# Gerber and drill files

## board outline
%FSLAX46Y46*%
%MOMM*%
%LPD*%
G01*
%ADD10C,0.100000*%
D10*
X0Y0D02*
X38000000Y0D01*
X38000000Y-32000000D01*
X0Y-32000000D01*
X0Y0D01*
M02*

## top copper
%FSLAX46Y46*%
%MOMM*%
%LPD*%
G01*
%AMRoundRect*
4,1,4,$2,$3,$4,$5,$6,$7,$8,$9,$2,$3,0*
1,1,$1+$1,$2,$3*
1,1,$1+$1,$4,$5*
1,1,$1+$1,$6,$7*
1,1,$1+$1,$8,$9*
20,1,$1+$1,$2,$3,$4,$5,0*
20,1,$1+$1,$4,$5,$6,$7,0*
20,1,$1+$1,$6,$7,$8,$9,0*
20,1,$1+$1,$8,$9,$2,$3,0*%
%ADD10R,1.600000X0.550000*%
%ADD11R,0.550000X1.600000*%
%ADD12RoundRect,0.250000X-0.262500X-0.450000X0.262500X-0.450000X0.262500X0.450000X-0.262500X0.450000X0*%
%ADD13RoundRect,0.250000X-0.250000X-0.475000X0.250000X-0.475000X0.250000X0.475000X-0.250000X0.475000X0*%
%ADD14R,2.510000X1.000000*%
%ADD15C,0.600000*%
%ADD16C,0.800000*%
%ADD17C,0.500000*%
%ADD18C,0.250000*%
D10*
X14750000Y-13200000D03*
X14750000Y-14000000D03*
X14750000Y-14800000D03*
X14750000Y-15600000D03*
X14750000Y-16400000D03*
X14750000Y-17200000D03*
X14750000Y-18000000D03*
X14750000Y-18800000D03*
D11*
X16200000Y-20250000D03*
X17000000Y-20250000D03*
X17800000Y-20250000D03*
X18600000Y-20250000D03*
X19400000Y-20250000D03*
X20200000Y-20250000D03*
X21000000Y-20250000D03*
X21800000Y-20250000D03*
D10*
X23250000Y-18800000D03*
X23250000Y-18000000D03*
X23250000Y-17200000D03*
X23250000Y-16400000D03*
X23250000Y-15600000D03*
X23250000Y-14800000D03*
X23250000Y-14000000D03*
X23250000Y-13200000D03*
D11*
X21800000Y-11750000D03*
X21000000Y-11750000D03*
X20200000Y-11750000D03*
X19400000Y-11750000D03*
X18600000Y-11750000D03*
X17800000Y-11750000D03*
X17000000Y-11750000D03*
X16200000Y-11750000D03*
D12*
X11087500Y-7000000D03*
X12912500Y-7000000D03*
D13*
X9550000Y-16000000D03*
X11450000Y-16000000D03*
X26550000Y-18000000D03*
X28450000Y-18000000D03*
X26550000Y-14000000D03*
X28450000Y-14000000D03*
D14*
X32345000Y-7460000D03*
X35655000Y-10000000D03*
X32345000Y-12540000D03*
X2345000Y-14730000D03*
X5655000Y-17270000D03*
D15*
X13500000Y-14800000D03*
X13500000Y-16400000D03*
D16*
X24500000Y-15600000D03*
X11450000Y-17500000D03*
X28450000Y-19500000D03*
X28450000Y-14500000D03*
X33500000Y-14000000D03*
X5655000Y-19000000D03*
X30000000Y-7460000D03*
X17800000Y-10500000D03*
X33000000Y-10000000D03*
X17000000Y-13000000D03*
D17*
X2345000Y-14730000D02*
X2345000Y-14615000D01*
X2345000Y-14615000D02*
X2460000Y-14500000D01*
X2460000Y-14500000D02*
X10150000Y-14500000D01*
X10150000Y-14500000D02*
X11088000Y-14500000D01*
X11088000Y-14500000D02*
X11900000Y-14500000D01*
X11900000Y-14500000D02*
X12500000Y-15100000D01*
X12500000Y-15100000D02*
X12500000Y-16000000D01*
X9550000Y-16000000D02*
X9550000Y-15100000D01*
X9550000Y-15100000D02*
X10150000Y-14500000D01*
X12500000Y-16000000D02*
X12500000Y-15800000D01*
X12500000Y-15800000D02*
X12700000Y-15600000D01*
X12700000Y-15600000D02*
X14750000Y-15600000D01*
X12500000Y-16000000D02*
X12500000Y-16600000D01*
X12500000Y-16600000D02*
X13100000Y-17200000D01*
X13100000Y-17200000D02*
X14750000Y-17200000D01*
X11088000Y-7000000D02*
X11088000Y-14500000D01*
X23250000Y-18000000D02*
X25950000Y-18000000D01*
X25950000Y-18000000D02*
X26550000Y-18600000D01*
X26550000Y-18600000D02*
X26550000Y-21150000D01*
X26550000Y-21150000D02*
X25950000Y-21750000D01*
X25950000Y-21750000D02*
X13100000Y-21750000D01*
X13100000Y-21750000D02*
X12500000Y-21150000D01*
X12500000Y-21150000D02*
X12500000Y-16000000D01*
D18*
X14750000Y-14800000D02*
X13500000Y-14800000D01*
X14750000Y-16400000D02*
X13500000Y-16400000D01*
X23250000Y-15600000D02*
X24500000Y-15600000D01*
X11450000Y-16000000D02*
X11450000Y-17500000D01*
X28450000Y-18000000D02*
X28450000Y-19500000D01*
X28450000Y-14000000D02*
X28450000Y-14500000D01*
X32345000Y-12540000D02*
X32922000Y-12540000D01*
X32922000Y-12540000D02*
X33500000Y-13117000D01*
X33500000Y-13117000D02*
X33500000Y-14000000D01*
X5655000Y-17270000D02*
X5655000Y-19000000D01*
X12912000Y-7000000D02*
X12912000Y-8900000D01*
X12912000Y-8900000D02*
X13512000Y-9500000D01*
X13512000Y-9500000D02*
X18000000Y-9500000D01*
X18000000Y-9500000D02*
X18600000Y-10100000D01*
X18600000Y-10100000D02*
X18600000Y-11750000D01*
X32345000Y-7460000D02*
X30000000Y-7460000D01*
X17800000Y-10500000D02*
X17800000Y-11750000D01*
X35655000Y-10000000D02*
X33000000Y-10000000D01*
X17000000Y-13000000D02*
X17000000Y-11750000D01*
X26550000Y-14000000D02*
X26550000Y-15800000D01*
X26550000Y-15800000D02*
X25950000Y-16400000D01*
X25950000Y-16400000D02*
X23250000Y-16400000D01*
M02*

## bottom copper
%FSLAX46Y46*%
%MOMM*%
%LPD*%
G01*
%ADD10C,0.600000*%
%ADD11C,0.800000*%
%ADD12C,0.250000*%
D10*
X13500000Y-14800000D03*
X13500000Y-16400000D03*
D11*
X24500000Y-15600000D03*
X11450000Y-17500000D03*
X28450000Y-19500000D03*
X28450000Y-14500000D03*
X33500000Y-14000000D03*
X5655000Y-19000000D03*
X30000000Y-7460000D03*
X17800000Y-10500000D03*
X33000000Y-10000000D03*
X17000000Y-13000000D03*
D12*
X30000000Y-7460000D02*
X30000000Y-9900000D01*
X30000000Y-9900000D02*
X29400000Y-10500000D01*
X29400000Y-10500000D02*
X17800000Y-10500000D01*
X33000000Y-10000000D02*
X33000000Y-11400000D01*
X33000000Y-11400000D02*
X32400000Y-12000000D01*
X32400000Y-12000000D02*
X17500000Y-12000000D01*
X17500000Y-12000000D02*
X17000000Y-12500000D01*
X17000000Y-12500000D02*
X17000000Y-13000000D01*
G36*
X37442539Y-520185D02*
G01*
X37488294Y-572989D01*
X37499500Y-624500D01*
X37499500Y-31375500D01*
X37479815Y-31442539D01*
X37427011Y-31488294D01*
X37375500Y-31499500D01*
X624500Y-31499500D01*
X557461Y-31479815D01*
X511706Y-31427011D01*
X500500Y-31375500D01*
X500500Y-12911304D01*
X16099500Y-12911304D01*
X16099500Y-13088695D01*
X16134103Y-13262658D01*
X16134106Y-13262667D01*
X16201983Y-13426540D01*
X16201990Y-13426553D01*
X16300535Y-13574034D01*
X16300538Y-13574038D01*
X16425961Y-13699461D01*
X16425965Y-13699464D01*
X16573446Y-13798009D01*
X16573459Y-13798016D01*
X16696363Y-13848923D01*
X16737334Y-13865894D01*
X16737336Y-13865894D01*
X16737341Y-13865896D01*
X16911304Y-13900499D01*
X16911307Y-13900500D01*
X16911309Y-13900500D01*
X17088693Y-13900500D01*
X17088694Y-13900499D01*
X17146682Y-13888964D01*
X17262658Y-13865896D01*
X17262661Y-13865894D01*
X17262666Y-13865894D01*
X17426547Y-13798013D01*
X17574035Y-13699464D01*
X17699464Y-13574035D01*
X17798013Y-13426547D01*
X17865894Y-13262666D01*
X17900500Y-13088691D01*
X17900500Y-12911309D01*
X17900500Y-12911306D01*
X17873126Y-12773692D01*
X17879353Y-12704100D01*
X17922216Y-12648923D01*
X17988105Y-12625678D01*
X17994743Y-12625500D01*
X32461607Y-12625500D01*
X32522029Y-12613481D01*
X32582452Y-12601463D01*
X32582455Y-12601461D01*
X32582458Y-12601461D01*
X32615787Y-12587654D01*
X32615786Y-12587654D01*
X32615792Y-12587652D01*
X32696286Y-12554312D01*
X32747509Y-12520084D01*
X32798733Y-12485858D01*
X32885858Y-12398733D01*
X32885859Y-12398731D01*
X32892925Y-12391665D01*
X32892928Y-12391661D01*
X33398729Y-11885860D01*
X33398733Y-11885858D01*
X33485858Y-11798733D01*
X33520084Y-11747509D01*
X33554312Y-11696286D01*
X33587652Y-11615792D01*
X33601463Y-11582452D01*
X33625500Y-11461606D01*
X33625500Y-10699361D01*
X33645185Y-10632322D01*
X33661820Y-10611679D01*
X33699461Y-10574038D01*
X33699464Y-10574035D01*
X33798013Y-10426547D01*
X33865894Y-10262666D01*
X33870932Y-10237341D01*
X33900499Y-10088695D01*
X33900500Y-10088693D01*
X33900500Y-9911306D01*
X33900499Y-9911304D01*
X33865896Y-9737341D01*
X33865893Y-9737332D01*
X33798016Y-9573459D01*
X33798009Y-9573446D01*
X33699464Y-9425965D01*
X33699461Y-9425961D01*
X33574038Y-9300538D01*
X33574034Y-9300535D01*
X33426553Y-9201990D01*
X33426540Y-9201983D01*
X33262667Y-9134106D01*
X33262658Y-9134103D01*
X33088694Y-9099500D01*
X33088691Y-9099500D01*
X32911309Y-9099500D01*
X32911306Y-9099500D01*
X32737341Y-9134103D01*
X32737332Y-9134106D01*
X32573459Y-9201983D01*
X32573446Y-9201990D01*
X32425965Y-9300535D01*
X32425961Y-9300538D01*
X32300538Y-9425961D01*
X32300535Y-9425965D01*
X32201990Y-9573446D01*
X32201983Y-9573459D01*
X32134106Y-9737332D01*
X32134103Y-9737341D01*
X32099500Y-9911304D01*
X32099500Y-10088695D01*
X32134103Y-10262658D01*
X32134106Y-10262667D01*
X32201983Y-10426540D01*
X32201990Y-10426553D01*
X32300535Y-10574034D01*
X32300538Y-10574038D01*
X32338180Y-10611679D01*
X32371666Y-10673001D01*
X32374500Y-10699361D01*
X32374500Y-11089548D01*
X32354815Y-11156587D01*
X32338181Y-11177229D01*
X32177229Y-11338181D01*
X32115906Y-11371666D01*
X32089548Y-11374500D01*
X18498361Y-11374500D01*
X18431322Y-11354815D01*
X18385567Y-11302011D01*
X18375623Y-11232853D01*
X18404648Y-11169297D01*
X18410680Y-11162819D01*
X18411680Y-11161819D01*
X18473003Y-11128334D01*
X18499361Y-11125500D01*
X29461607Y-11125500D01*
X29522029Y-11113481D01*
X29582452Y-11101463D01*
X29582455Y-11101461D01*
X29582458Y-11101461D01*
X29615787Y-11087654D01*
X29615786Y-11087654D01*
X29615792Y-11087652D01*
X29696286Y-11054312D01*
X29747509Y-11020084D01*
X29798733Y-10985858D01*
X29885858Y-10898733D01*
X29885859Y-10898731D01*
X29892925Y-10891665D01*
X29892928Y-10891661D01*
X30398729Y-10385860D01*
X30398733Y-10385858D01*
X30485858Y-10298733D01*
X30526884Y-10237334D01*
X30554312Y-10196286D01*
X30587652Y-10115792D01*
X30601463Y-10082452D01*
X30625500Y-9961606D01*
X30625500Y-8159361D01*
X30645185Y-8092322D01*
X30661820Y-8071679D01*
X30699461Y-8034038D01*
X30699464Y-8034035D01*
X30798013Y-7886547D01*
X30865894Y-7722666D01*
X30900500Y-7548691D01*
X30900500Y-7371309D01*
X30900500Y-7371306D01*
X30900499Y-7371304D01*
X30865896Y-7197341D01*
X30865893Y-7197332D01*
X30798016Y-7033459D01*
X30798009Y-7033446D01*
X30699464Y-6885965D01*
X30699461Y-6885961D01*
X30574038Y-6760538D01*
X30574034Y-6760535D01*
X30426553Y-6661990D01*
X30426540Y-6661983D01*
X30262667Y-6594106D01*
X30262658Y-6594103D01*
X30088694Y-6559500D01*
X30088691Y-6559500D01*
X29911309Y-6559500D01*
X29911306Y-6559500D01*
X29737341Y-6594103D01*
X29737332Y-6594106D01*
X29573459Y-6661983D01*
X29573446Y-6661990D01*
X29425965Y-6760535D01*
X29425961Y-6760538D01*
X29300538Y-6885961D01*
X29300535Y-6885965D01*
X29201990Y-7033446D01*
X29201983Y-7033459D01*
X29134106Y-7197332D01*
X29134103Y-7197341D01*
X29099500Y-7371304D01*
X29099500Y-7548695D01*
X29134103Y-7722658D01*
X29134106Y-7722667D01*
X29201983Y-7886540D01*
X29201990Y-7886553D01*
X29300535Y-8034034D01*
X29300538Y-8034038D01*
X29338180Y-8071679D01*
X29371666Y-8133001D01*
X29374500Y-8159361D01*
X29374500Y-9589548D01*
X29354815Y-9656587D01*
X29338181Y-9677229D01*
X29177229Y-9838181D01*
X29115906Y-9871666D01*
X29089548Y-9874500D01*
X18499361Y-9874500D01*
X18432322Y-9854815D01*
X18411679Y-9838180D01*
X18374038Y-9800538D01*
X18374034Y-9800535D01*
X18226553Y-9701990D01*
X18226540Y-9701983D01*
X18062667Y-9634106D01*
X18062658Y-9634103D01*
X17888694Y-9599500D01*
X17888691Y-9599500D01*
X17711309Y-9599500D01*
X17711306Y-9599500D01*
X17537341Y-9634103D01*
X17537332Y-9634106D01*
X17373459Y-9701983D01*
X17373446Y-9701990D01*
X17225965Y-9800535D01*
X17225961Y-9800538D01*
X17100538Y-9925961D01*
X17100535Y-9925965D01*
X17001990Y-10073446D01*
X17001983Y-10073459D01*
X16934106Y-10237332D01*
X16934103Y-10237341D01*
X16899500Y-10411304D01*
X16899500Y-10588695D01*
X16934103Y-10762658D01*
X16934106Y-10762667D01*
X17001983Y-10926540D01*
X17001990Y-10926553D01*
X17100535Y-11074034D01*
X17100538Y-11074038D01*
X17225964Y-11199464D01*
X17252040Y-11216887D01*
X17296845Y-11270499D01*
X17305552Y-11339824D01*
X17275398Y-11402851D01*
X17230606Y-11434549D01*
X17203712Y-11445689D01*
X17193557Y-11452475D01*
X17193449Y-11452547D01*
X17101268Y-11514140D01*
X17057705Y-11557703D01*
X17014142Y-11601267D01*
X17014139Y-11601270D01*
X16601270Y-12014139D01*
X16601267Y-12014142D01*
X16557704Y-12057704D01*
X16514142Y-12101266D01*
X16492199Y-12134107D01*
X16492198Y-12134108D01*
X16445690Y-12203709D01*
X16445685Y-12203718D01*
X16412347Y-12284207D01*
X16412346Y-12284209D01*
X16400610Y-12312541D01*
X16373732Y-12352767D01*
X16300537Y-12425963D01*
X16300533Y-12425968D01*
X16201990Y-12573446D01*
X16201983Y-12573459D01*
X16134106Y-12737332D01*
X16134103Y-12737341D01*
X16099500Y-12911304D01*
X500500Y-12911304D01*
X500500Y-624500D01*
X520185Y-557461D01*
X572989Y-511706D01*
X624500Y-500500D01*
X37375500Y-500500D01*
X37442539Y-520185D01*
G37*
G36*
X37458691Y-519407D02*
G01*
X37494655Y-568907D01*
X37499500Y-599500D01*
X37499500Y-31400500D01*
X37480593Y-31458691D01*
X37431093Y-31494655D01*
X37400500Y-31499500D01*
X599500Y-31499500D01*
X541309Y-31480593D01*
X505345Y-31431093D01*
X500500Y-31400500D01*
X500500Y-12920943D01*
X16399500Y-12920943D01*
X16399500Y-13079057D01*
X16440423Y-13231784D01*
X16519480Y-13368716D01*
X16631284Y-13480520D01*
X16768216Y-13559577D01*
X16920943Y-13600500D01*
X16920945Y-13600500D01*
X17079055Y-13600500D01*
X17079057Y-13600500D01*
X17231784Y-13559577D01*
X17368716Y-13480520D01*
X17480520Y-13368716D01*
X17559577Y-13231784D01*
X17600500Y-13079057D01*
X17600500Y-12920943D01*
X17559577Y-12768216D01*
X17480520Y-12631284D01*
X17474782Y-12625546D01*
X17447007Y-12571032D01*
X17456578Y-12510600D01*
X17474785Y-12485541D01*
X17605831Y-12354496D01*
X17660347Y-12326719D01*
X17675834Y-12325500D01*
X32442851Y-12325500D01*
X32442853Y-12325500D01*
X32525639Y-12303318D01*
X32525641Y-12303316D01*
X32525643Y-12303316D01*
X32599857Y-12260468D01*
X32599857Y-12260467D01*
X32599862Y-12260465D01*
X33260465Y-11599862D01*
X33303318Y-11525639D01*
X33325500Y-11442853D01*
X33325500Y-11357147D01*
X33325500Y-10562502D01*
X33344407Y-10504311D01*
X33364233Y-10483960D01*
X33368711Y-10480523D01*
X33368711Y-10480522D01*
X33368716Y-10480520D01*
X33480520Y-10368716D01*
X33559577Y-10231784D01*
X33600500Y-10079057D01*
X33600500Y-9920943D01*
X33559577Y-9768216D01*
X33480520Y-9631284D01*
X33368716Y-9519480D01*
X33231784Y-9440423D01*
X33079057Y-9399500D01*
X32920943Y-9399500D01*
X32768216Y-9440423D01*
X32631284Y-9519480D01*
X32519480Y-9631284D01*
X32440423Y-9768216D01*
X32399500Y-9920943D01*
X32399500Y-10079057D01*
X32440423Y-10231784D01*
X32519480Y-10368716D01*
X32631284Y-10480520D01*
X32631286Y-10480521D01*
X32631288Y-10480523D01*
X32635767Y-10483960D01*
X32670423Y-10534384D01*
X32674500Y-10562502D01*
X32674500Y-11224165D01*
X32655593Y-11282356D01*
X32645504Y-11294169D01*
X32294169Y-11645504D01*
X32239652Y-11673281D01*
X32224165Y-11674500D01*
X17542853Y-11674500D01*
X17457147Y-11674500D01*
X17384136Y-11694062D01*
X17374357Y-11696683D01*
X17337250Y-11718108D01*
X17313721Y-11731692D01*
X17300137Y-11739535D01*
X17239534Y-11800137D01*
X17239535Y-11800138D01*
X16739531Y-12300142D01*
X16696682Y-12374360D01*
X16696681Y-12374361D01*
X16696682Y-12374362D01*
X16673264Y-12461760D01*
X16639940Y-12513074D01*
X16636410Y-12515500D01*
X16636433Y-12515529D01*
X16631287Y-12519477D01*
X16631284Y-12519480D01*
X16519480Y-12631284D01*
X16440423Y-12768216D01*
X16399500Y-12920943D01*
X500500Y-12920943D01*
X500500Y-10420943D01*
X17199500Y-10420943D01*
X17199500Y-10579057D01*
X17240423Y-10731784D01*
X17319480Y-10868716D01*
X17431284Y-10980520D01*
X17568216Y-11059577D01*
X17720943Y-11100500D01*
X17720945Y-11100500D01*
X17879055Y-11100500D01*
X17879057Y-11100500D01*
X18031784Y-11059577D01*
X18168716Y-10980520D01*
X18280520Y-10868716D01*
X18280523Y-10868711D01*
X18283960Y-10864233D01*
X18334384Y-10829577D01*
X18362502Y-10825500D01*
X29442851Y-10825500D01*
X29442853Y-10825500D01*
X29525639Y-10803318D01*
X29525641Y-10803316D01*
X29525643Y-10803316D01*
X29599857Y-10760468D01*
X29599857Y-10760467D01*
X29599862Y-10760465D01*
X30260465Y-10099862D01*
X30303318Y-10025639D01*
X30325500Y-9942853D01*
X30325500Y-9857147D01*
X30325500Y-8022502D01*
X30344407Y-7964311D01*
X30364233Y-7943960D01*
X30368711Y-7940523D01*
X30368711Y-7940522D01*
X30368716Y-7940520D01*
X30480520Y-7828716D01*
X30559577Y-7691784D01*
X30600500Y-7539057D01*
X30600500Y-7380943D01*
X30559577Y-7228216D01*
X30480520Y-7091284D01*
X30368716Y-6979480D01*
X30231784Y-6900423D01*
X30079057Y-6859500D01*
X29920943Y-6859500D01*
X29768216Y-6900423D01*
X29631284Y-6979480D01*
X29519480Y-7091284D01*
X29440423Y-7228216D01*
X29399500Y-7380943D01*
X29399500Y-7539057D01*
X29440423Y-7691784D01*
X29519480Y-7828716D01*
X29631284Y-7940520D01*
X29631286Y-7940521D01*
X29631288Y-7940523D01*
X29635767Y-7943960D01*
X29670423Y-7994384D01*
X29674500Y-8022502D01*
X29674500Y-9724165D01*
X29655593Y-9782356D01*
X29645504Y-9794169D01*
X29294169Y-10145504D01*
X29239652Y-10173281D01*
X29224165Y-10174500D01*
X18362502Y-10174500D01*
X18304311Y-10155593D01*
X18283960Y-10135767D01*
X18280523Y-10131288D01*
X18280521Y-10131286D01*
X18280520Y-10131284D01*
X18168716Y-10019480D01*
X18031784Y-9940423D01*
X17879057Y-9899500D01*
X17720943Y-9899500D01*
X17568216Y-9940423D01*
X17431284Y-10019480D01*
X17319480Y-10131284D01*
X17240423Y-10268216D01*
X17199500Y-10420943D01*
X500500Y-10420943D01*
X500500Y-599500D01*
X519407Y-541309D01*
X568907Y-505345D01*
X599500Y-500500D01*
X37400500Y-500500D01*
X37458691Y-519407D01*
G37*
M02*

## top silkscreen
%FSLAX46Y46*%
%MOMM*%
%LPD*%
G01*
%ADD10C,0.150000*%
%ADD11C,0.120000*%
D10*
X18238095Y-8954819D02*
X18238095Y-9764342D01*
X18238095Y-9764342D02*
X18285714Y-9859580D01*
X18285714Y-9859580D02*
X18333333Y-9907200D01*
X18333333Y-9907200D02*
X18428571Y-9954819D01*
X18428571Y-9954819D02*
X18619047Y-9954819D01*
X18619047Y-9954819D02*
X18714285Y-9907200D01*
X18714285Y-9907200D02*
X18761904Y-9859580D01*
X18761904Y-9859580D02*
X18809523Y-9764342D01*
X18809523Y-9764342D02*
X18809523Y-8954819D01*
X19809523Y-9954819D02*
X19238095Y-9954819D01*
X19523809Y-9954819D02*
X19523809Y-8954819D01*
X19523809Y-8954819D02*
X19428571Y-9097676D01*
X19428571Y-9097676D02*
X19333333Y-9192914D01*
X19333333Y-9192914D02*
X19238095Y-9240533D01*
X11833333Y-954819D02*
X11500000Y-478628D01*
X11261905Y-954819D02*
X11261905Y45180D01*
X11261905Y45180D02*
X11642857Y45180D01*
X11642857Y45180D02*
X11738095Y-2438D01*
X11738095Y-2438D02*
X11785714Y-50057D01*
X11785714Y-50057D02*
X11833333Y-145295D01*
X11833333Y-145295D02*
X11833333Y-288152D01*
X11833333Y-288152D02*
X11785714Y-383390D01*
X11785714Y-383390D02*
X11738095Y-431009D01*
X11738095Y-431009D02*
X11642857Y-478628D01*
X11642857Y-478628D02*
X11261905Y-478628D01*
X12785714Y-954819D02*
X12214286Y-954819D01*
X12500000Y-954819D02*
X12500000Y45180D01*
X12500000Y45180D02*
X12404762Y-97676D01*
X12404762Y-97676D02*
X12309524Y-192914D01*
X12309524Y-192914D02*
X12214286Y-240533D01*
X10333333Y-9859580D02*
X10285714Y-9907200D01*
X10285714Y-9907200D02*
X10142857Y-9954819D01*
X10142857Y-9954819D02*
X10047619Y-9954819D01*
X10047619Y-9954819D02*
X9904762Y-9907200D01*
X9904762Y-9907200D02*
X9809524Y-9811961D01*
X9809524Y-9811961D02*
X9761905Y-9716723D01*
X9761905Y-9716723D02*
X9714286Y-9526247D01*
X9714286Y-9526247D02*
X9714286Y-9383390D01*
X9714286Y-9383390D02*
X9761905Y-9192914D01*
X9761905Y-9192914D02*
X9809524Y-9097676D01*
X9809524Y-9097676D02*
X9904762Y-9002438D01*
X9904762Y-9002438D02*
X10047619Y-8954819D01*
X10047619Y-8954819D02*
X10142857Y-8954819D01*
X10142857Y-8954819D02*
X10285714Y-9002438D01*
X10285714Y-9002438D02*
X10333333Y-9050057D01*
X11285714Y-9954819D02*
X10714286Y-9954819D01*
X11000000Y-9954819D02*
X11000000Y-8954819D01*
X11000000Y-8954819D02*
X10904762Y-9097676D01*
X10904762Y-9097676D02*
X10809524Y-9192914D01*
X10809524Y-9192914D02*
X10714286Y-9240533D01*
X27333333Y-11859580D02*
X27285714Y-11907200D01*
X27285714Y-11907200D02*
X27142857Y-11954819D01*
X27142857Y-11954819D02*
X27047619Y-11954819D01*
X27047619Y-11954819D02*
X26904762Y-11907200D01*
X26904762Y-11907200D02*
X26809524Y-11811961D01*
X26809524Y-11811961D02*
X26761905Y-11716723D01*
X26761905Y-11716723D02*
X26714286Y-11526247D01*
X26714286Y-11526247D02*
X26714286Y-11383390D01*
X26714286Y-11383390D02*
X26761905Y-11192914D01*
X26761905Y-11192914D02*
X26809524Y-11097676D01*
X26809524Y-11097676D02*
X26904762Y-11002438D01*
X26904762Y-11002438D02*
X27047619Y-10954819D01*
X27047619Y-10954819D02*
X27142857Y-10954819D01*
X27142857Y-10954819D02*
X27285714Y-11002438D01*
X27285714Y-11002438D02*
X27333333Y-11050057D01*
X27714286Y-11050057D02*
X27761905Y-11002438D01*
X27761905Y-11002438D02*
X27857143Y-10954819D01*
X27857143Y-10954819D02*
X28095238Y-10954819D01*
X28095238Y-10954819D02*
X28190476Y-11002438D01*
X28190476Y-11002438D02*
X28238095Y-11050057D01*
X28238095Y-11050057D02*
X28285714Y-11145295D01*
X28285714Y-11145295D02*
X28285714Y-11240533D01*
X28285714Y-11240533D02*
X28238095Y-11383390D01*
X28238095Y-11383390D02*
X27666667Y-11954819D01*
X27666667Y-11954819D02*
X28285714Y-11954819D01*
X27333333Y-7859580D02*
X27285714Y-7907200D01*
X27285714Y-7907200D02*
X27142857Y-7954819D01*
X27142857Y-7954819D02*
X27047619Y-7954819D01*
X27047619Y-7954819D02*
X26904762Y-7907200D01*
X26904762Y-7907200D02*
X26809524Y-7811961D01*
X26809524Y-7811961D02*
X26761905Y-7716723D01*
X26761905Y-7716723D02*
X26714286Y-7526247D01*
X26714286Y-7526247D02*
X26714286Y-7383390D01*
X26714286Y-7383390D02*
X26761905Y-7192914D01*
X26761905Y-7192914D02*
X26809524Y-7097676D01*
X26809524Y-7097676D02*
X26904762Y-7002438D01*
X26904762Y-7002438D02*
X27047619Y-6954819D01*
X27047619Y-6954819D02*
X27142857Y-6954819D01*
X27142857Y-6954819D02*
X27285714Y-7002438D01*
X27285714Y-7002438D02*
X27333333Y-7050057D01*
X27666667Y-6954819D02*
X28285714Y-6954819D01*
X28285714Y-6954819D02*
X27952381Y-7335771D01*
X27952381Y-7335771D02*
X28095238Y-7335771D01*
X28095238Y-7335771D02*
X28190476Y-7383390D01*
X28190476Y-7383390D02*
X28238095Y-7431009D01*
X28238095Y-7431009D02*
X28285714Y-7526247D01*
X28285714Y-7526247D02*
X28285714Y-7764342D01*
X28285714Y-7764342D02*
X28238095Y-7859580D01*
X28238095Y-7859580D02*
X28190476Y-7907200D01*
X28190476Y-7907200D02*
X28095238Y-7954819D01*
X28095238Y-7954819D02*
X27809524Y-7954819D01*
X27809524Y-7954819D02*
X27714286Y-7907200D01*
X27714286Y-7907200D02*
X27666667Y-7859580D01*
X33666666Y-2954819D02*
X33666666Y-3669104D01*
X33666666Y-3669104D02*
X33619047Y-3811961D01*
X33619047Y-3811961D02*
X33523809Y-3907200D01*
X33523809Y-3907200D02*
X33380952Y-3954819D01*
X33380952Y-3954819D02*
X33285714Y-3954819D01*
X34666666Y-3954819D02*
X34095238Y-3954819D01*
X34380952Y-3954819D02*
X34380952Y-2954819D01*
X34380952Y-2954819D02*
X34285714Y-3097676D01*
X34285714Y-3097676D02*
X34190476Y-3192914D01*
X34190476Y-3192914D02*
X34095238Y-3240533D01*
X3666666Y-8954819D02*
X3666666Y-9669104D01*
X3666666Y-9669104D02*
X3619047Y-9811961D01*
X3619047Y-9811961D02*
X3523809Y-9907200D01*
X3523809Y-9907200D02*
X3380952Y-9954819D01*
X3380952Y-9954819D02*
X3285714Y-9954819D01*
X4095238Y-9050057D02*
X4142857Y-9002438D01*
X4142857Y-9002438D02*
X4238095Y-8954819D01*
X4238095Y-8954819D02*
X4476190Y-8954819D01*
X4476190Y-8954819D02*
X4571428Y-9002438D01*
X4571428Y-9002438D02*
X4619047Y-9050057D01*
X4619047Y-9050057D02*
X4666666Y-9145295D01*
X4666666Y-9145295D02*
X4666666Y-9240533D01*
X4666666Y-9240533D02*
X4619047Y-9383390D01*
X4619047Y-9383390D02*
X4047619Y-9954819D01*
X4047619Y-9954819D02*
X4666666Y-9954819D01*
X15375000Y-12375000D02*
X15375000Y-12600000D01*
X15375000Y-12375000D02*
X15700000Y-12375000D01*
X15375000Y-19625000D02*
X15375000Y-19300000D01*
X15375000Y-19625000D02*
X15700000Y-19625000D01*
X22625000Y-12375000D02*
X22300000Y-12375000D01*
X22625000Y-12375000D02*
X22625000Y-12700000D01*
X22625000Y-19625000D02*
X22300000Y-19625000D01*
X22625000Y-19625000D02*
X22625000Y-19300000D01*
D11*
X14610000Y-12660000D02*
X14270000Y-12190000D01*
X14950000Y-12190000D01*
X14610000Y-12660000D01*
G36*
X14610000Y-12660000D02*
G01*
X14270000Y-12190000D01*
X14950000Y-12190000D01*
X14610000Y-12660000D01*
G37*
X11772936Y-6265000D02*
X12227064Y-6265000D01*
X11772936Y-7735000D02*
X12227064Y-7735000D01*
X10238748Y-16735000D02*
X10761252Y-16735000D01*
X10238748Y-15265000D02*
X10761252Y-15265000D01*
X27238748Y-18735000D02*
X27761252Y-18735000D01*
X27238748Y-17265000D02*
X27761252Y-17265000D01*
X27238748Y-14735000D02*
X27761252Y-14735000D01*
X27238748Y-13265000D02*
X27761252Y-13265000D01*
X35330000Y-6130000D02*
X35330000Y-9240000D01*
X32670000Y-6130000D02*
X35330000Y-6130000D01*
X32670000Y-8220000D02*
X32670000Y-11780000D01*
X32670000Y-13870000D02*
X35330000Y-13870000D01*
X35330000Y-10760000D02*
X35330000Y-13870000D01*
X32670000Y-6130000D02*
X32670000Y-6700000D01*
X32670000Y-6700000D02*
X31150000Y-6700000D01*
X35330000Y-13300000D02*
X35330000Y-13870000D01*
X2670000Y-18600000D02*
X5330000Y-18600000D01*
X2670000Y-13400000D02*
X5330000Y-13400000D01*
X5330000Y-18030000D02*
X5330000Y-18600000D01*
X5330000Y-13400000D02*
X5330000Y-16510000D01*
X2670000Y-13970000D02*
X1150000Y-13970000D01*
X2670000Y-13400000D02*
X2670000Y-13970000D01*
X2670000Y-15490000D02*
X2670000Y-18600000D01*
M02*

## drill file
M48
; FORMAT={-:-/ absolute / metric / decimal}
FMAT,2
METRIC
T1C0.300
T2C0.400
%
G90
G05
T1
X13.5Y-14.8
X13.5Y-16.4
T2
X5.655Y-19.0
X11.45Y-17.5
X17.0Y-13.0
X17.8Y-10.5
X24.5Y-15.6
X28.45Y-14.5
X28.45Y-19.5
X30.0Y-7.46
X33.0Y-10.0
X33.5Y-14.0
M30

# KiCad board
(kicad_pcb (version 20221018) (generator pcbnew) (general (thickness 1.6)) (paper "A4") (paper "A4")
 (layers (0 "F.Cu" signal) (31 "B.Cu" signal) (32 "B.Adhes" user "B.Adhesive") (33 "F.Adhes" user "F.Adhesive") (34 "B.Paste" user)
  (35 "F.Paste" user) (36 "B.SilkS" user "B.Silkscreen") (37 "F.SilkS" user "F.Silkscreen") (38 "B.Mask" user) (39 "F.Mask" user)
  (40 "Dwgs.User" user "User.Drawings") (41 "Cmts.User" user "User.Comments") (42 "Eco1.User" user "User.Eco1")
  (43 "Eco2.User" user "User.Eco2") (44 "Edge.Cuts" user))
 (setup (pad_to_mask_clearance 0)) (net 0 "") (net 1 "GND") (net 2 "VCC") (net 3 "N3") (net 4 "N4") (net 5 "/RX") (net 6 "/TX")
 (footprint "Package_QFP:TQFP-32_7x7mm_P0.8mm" (layer "F.Cu") (at 19 16) (layer "F.Cu")
  (fp_line (start -3.625 -3.625) (end -3.625 -3.4) (stroke (width 0.15) (type solid)) (layer "F.SilkS"))
  (fp_line (start -3.625 -3.625) (end -3.3 -3.625) (stroke (width 0.15) (type solid)) (layer "F.SilkS"))
  (fp_line (start -3.625 3.625) (end -3.625 3.3) (stroke (width 0.15) (type solid)) (layer "F.SilkS"))
  (fp_line (start -3.625 3.625) (end -3.3 3.625) (stroke (width 0.15) (type solid)) (layer "F.SilkS"))
  (fp_line (start 3.625 -3.625) (end 3.3 -3.625) (stroke (width 0.15) (type solid)) (layer "F.SilkS"))
  (fp_line (start 3.625 -3.625) (end 3.625 -3.3) (stroke (width 0.15) (type solid)) (layer "F.SilkS"))
  (fp_line (start 3.625 3.625) (end 3.3 3.625) (stroke (width 0.15) (type solid)) (layer "F.SilkS"))
  (fp_line (start 3.625 3.625) (end 3.625 3.3) (stroke (width 0.15) (type solid)) (layer "F.SilkS"))
  (fp_poly
   (pts (xy -4.39 -3.34) (xy -4.73 -3.81) (xy -4.05 -3.81) (xy -4.39 -3.34)) (stroke (width 0.12) (type solid)) (fill solid)
   (layer "F.SilkS"))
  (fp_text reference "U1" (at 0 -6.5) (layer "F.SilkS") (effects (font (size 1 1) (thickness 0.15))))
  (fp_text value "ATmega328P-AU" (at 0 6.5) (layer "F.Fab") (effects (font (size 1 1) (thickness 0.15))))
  (pad "1" smd rect (at -4.25 -2.8) (size 1.6 0.55) (layers "F.Cu" "F.Paste" "F.Mask") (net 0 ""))
  (pad "2" smd rect (at -4.25 -2) (size 1.6 0.55) (layers "F.Cu" "F.Paste" "F.Mask") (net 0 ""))
  (pad "3" smd rect (at -4.25 -1.2) (size 1.6 0.55) (layers "F.Cu" "F.Paste" "F.Mask") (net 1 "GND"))
  (pad "4" smd rect (at -4.25 -0.4) (size 1.6 0.55) (layers "F.Cu" "F.Paste" "F.Mask") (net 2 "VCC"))
  (pad "5" smd rect (at -4.25 0.4) (size 1.6 0.55) (layers "F.Cu" "F.Paste" "F.Mask") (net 1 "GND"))
  (pad "6" smd rect (at -4.25 1.2) (size 1.6 0.55) (layers "F.Cu" "F.Paste" "F.Mask") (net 2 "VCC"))
  (pad "7" smd rect (at -4.25 2) (size 1.6 0.55) (layers "F.Cu" "F.Paste" "F.Mask") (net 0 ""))
  (pad "8" smd rect (at -4.25 2.8) (size 1.6 0.55) (layers "F.Cu" "F.Paste" "F.Mask") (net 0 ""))
  (pad "9" smd rect (at -2.8 4.25 90) (size 1.6 0.55) (layers "F.Cu" "F.Paste" "F.Mask") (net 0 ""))
  (pad "10" smd rect (at -2 4.25 90) (size 1.6 0.55) (layers "F.Cu" "F.Paste" "F.Mask") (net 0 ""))
  (pad "11" smd rect (at -1.2 4.25 90) (size 1.6 0.55) (layers "F.Cu" "F.Paste" "F.Mask") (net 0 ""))
  (pad "12" smd rect (at -0.4 4.25 90) (size 1.6 0.55) (layers "F.Cu" "F.Paste" "F.Mask") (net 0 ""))
  (pad "13" smd rect (at 0.4 4.25 90) (size 1.6 0.55) (layers "F.Cu" "F.Paste" "F.Mask") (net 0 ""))
  (pad "14" smd rect (at 1.2 4.25 90) (size 1.6 0.55) (layers "F.Cu" "F.Paste" "F.Mask") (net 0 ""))
  (pad "15" smd rect (at 2 4.25 90) (size 1.6 0.55) (layers "F.Cu" "F.Paste" "F.Mask") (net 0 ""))
  (pad "16" smd rect (at 2.8 4.25 90) (size 1.6 0.55) (layers "F.Cu" "F.Paste" "F.Mask") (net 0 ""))
  (pad "17" smd rect (at 4.25 2.8) (size 1.6 0.55) (layers "F.Cu" "F.Paste" "F.Mask") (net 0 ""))
  (pad "18" smd rect (at 4.25 2) (size 1.6 0.55) (layers "F.Cu" "F.Paste" "F.Mask") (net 2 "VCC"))
  (pad "19" smd rect (at 4.25 1.2) (size 1.6 0.55) (layers "F.Cu" "F.Paste" "F.Mask") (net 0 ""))
  (pad "20" smd rect (at 4.25 0.4) (size 1.6 0.55) (layers "F.Cu" "F.Paste" "F.Mask") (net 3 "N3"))
  (pad "21" smd rect (at 4.25 -0.4) (size 1.6 0.55) (layers "F.Cu" "F.Paste" "F.Mask") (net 1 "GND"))
  (pad "22" smd rect (at 4.25 -1.2) (size 1.6 0.55) (layers "F.Cu" "F.Paste" "F.Mask") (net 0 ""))
  (pad "23" smd rect (at 4.25 -2) (size 1.6 0.55) (layers "F.Cu" "F.Paste" "F.Mask") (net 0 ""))
  (pad "24" smd rect (at 4.25 -2.8) (size 1.6 0.55) (layers "F.Cu" "F.Paste" "F.Mask") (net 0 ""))
  (pad "25" smd rect (at 2.8 -4.25 90) (size 1.6 0.55) (layers "F.Cu" "F.Paste" "F.Mask") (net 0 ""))
  (pad "26" smd rect (at 2 -4.25 90) (size 1.6 0.55) (layers "F.Cu" "F.Paste" "F.Mask") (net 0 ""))
  (pad "27" smd rect (at 1.2 -4.25 90) (size 1.6 0.55) (layers "F.Cu" "F.Paste" "F.Mask") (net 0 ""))
  (pad "28" smd rect (at 0.4 -4.25 90) (size 1.6 0.55) (layers "F.Cu" "F.Paste" "F.Mask") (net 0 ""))
  (pad "29" smd rect (at -0.4 -4.25 90) (size 1.6 0.55) (layers "F.Cu" "F.Paste" "F.Mask") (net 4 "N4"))
  (pad "30" smd rect (at -1.2 -4.25 90) (size 1.6 0.55) (layers "F.Cu" "F.Paste" "F.Mask") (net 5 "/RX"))
  (pad "31" smd rect (at -2 -4.25 90) (size 1.6 0.55) (layers "F.Cu" "F.Paste" "F.Mask") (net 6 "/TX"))
  (pad "32" smd rect (at -2.8 -4.25 90) (size 1.6 0.55) (layers "F.Cu" "F.Paste" "F.Mask") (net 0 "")))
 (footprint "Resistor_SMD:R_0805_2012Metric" (layer "F.Cu") (at 12 7) (layer "F.Cu")
  (fp_line (start -0.227064 -0.735) (end 0.227064 -0.735) (layer "F.SilkS") (width 0.12))
  (fp_line (start -0.227064 0.735) (end 0.227064 0.735) (layer "F.SilkS") (width 0.12))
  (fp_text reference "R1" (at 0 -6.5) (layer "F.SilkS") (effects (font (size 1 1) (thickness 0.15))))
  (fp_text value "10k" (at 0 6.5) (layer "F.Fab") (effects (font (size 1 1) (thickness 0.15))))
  (pad "1" smd roundrect (at -0.9125 0) (size 1.025 1.4) (layers "F.Cu" "F.Paste" "F.Mask") (roundrect_rratio 0.243902) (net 2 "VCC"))
  (pad "2" smd roundrect (at 0.9125 0) (size 1.025 1.4) (layers "F.Cu" "F.Paste" "F.Mask") (roundrect_rratio 0.243902) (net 4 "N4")))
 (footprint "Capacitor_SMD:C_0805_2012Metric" (layer "F.Cu") (at 10.5 16) (layer "F.Cu")
  (fp_line (start -0.261252 0.735) (end 0.261252 0.735) (layer "F.SilkS") (width 0.12))
  (fp_line (start -0.261252 -0.735) (end 0.261252 -0.735) (layer "F.SilkS") (width 0.12))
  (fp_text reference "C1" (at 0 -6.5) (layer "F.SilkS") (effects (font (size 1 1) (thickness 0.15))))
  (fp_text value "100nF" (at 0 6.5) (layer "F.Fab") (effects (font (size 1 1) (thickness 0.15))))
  (pad "1" smd roundrect (at -0.95 0) (size 1 1.45) (layers "F.Cu" "F.Paste" "F.Mask") (roundrect_rratio 0.25) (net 2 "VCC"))
  (pad "2" smd roundrect (at 0.95 0) (size 1 1.45) (layers "F.Cu" "F.Paste" "F.Mask") (roundrect_rratio 0.25) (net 1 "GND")))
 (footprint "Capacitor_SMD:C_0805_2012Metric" (layer "F.Cu") (at 27.5 18) (layer "F.Cu")
  (fp_line (start -0.261252 0.735) (end 0.261252 0.735) (layer "F.SilkS") (width 0.12))
  (fp_line (start -0.261252 -0.735) (end 0.261252 -0.735) (layer "F.SilkS") (width 0.12))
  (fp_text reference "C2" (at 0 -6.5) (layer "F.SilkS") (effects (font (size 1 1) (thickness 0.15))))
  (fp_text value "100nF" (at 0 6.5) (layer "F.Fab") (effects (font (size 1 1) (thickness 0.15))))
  (pad "1" smd roundrect (at -0.95 0) (size 1 1.45) (layers "F.Cu" "F.Paste" "F.Mask") (roundrect_rratio 0.25) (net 2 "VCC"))
  (pad "2" smd roundrect (at 0.95 0) (size 1 1.45) (layers "F.Cu" "F.Paste" "F.Mask") (roundrect_rratio 0.25) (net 1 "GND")))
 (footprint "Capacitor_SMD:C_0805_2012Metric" (layer "F.Cu") (at 27.5 14) (layer "F.Cu")
  (fp_line (start -0.261252 0.735) (end 0.261252 0.735) (layer "F.SilkS") (width 0.12))
  (fp_line (start -0.261252 -0.735) (end 0.261252 -0.735) (layer "F.SilkS") (width 0.12))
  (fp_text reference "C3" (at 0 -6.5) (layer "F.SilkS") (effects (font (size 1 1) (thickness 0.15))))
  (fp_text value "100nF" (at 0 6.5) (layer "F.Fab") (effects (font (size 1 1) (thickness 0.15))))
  (pad "1" smd roundrect (at -0.95 0) (size 1 1.45) (layers "F.Cu" "F.Paste" "F.Mask") (roundrect_rratio 0.25) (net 3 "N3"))
  (pad "2" smd roundrect (at 0.95 0) (size 1 1.45) (layers "F.Cu" "F.Paste" "F.Mask") (roundrect_rratio 0.25) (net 1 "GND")))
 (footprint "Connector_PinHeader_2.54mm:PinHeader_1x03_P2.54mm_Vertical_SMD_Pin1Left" (layer "F.Cu") (at 34 10) (layer "F.Cu")
  (fp_line (start 1.33 -3.87) (end 1.33 -0.76) (layer "F.SilkS") (width 0.12))
  (fp_line (start -1.33 -3.87) (end 1.33 -3.87) (layer "F.SilkS") (width 0.12))
  (fp_line (start -1.33 -1.78) (end -1.33 1.78) (layer "F.SilkS") (width 0.12))
  (fp_line (start -1.33 3.87) (end 1.33 3.87) (layer "F.SilkS") (width 0.12))
  (fp_line (start 1.33 0.76) (end 1.33 3.87) (layer "F.SilkS") (width 0.12))
  (fp_line (start -1.33 -3.87) (end -1.33 -3.3) (layer "F.SilkS") (width 0.12))
  (fp_line (start -1.33 -3.3) (end -2.85 -3.3) (layer "F.SilkS") (width 0.12))
  (fp_line (start 1.33 3.3) (end 1.33 3.87) (layer "F.SilkS") (width 0.12))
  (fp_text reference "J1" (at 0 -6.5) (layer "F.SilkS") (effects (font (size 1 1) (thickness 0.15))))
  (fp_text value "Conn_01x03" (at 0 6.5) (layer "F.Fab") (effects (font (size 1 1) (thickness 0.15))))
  (pad "1" smd rect (at -1.655 -2.54) (size 2.51 1) (layers "F.Cu" "F.Paste" "F.Mask") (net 5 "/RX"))
  (pad "2" smd rect (at 1.655 0) (size 2.51 1) (layers "F.Cu" "F.Paste" "F.Mask") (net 6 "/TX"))
  (pad "3" smd rect (at -1.655 2.54) (size 2.51 1) (layers "F.Cu" "F.Paste" "F.Mask") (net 1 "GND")))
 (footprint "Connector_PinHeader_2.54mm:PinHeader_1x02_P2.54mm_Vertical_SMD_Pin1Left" (layer "F.Cu") (at 4 16) (layer "F.Cu")
  (fp_line (start -1.33 2.6) (end 1.33 2.6) (layer "F.SilkS") (width 0.12))
  (fp_line (start -1.33 -2.6) (end 1.33 -2.6) (layer "F.SilkS") (width 0.12))
  (fp_line (start 1.33 2.03) (end 1.33 2.6) (layer "F.SilkS") (width 0.12))
  (fp_line (start 1.33 -2.6) (end 1.33 0.51) (layer "F.SilkS") (width 0.12))
  (fp_line (start -1.33 -2.03) (end -2.85 -2.03) (layer "F.SilkS") (width 0.12))
  (fp_line (start -1.33 -2.6) (end -1.33 -2.03) (layer "F.SilkS") (width 0.12))
  (fp_line (start -1.33 -0.51) (end -1.33 2.6) (layer "F.SilkS") (width 0.12))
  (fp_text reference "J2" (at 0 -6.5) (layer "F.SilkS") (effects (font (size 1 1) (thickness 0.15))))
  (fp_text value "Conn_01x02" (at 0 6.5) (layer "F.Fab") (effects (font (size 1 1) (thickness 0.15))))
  (pad "1" smd rect (at -1.655 -1.27) (size 2.51 1) (layers "F.Cu" "F.Paste" "F.Mask") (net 2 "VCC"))
  (pad "2" smd rect (at 1.655 1.27) (size 2.51 1) (layers "F.Cu" "F.Paste" "F.Mask") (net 1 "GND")))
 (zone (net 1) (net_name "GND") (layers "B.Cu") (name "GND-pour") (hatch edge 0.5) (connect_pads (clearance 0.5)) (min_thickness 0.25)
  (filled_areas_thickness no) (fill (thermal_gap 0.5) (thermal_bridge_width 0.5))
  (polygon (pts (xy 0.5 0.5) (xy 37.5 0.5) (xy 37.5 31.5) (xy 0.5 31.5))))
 (gr_rect (start 0 0) (end 38 32) (layer "Edge.Cuts") (width 0.1))
 (segment (start 2.345 14.730) (end 2.345 14.615) (width 0.5) (layer "F.Cu") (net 2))
 (segment (start 2.345 14.615) (end 2.460 14.500) (width 0.5) (layer "F.Cu") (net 2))
 (segment (start 2.460 14.500) (end 10.150 14.500) (width 0.5) (layer "F.Cu") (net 2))
 (segment (start 10.150 14.500) (end 11.088 14.500) (width 0.5) (layer "F.Cu") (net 2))
 (segment (start 11.088 14.500) (end 11.900 14.500) (width 0.5) (layer "F.Cu") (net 2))
 (segment (start 11.900 14.500) (end 12.500 15.100) (width 0.5) (layer "F.Cu") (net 2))
 (segment (start 12.500 15.100) (end 12.500 16.000) (width 0.5) (layer "F.Cu") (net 2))
 (segment (start 9.550 16.000) (end 9.550 15.100) (width 0.5) (layer "F.Cu") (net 2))
 (segment (start 9.550 15.100) (end 10.150 14.500) (width 0.5) (layer "F.Cu") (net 2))
 (segment (start 12.500 16.000) (end 12.500 15.800) (width 0.5) (layer "F.Cu") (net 2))
 (segment (start 12.500 15.800) (end 12.700 15.600) (width 0.5) (layer "F.Cu") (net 2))
 (segment (start 12.700 15.600) (end 14.750 15.600) (width 0.5) (layer "F.Cu") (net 2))
 (segment (start 12.500 16.000) (end 12.500 16.600) (width 0.5) (layer "F.Cu") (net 2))
 (segment (start 12.500 16.600) (end 13.100 17.200) (width 0.5) (layer "F.Cu") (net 2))
 (segment (start 13.100 17.200) (end 14.750 17.200) (width 0.5) (layer "F.Cu") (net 2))
 (segment (start 11.088 7.000) (end 11.088 14.500) (width 0.5) (layer "F.Cu") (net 2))
 (segment (start 23.250 18.000) (end 25.950 18.000) (width 0.5) (layer "F.Cu") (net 2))
 (segment (start 25.950 18.000) (end 26.550 18.600) (width 0.5) (layer "F.Cu") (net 2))
 (segment (start 26.550 18.600) (end 26.550 21.150) (width 0.5) (layer "F.Cu") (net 2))
 (segment (start 26.550 21.150) (end 25.950 21.750) (width 0.5) (layer "F.Cu") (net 2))
 (segment (start 25.950 21.750) (end 13.100 21.750) (width 0.5) (layer "F.Cu") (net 2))
 (segment (start 13.100 21.750) (end 12.500 21.150) (width 0.5) (layer "F.Cu") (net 2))
 (segment (start 12.500 21.150) (end 12.500 16.000) (width 0.5) (layer "F.Cu") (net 2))
 (segment (start 14.750 14.800) (end 13.500 14.800) (width 0.25) (layer "F.Cu") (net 1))
 (via (at 13.500 14.800) (size 0.6) (drill 0.3) (layers "F.Cu" "B.Cu") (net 1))
 (segment (start 14.750 16.400) (end 13.500 16.400) (width 0.25) (layer "F.Cu") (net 1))
 (via (at 13.500 16.400) (size 0.6) (drill 0.3) (layers "F.Cu" "B.Cu") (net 1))
 (segment (start 23.250 15.600) (end 24.500 15.600) (width 0.25) (layer "F.Cu") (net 1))
 (via (at 24.500 15.600) (size 0.8) (drill 0.4) (layers "F.Cu" "B.Cu") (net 1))
 (segment (start 11.450 16.000) (end 11.450 17.500) (width 0.25) (layer "F.Cu") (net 1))
 (via (at 11.450 17.500) (size 0.8) (drill 0.4) (layers "F.Cu" "B.Cu") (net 1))
 (segment (start 28.450 18.000) (end 28.450 19.500) (width 0.25) (layer "F.Cu") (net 1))
 (via (at 28.450 19.500) (size 0.8) (drill 0.4) (layers "F.Cu" "B.Cu") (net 1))
 (segment (start 28.450 14.000) (end 28.450 14.500) (width 0.25) (layer "F.Cu") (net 1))
 (via (at 28.450 14.500) (size 0.8) (drill 0.4) (layers "F.Cu" "B.Cu") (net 1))
 (segment (start 32.345 12.540) (end 32.922 12.540) (width 0.25) (layer "F.Cu") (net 1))
 (segment (start 32.922 12.540) (end 33.500 13.117) (width 0.25) (layer "F.Cu") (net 1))
 (segment (start 33.500 13.117) (end 33.500 14.000) (width 0.25) (layer "F.Cu") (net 1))
 (via (at 33.500 14.000) (size 0.8) (drill 0.4) (layers "F.Cu" "B.Cu") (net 1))
 (segment (start 5.655 17.270) (end 5.655 19.000) (width 0.25) (layer "F.Cu") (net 1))
 (via (at 5.655 19.000) (size 0.8) (drill 0.4) (layers "F.Cu" "B.Cu") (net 1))
 (segment (start 12.912 7.000) (end 12.912 8.900) (width 0.25) (layer "F.Cu") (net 4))
 (segment (start 12.912 8.900) (end 13.512 9.500) (width 0.25) (layer "F.Cu") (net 4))
 (segment (start 13.512 9.500) (end 18.000 9.500) (width 0.25) (layer "F.Cu") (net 4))
 (segment (start 18.000 9.500) (end 18.600 10.100) (width 0.25) (layer "F.Cu") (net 4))
 (segment (start 18.600 10.100) (end 18.600 11.750) (width 0.25) (layer "F.Cu") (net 4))
 (segment (start 32.345 7.460) (end 30.000 7.460) (width 0.25) (layer "F.Cu") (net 5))
 (via (at 30.000 7.460) (size 0.8) (drill 0.4) (layers "F.Cu" "B.Cu") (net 5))
 (segment (start 30.000 7.460) (end 30.000 9.900) (width 0.25) (layer "B.Cu") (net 5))
 (segment (start 30.000 9.900) (end 29.400 10.500) (width 0.25) (layer "B.Cu") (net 5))
 (segment (start 29.400 10.500) (end 17.800 10.500) (width 0.25) (layer "B.Cu") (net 5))
 (via (at 17.800 10.500) (size 0.8) (drill 0.4) (layers "F.Cu" "B.Cu") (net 5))
 (segment (start 17.800 10.500) (end 17.800 11.750) (width 0.25) (layer "F.Cu") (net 5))
 (segment (start 35.655 10.000) (end 33.000 10.000) (width 0.25) (layer "F.Cu") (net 6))
 (via (at 33.000 10.000) (size 0.8) (drill 0.4) (layers "F.Cu" "B.Cu") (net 6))
 (segment (start 33.000 10.000) (end 33.000 11.400) (width 0.25) (layer "B.Cu") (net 6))
 (segment (start 33.000 11.400) (end 32.400 12.000) (width 0.25) (layer "B.Cu") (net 6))
 (segment (start 32.400 12.000) (end 17.500 12.000) (width 0.25) (layer "B.Cu") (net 6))
 (segment (start 17.500 12.000) (end 17.000 12.500) (width 0.25) (layer "B.Cu") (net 6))
 (segment (start 17.000 12.500) (end 17.000 13.000) (width 0.25) (layer "B.Cu") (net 6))
 (via (at 17.000 13.000) (size 0.8) (drill 0.4) (layers "F.Cu" "B.Cu") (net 6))
 (segment (start 17.000 13.000) (end 17.000 11.750) (width 0.25) (layer "F.Cu") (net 6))
 (segment (start 26.550 14.000) (end 26.550 15.800) (width 0.25) (layer "F.Cu") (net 3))
 (segment (start 26.550 15.800) (end 25.950 16.400) (width 0.25) (layer "F.Cu") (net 3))
 (segment (start 25.950 16.400) (end 23.250 16.400) (width 0.25) (layer "F.Cu") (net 3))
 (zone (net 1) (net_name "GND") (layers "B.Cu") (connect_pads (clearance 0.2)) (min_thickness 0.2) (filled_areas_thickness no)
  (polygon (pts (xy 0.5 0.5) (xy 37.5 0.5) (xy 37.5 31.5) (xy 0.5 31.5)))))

